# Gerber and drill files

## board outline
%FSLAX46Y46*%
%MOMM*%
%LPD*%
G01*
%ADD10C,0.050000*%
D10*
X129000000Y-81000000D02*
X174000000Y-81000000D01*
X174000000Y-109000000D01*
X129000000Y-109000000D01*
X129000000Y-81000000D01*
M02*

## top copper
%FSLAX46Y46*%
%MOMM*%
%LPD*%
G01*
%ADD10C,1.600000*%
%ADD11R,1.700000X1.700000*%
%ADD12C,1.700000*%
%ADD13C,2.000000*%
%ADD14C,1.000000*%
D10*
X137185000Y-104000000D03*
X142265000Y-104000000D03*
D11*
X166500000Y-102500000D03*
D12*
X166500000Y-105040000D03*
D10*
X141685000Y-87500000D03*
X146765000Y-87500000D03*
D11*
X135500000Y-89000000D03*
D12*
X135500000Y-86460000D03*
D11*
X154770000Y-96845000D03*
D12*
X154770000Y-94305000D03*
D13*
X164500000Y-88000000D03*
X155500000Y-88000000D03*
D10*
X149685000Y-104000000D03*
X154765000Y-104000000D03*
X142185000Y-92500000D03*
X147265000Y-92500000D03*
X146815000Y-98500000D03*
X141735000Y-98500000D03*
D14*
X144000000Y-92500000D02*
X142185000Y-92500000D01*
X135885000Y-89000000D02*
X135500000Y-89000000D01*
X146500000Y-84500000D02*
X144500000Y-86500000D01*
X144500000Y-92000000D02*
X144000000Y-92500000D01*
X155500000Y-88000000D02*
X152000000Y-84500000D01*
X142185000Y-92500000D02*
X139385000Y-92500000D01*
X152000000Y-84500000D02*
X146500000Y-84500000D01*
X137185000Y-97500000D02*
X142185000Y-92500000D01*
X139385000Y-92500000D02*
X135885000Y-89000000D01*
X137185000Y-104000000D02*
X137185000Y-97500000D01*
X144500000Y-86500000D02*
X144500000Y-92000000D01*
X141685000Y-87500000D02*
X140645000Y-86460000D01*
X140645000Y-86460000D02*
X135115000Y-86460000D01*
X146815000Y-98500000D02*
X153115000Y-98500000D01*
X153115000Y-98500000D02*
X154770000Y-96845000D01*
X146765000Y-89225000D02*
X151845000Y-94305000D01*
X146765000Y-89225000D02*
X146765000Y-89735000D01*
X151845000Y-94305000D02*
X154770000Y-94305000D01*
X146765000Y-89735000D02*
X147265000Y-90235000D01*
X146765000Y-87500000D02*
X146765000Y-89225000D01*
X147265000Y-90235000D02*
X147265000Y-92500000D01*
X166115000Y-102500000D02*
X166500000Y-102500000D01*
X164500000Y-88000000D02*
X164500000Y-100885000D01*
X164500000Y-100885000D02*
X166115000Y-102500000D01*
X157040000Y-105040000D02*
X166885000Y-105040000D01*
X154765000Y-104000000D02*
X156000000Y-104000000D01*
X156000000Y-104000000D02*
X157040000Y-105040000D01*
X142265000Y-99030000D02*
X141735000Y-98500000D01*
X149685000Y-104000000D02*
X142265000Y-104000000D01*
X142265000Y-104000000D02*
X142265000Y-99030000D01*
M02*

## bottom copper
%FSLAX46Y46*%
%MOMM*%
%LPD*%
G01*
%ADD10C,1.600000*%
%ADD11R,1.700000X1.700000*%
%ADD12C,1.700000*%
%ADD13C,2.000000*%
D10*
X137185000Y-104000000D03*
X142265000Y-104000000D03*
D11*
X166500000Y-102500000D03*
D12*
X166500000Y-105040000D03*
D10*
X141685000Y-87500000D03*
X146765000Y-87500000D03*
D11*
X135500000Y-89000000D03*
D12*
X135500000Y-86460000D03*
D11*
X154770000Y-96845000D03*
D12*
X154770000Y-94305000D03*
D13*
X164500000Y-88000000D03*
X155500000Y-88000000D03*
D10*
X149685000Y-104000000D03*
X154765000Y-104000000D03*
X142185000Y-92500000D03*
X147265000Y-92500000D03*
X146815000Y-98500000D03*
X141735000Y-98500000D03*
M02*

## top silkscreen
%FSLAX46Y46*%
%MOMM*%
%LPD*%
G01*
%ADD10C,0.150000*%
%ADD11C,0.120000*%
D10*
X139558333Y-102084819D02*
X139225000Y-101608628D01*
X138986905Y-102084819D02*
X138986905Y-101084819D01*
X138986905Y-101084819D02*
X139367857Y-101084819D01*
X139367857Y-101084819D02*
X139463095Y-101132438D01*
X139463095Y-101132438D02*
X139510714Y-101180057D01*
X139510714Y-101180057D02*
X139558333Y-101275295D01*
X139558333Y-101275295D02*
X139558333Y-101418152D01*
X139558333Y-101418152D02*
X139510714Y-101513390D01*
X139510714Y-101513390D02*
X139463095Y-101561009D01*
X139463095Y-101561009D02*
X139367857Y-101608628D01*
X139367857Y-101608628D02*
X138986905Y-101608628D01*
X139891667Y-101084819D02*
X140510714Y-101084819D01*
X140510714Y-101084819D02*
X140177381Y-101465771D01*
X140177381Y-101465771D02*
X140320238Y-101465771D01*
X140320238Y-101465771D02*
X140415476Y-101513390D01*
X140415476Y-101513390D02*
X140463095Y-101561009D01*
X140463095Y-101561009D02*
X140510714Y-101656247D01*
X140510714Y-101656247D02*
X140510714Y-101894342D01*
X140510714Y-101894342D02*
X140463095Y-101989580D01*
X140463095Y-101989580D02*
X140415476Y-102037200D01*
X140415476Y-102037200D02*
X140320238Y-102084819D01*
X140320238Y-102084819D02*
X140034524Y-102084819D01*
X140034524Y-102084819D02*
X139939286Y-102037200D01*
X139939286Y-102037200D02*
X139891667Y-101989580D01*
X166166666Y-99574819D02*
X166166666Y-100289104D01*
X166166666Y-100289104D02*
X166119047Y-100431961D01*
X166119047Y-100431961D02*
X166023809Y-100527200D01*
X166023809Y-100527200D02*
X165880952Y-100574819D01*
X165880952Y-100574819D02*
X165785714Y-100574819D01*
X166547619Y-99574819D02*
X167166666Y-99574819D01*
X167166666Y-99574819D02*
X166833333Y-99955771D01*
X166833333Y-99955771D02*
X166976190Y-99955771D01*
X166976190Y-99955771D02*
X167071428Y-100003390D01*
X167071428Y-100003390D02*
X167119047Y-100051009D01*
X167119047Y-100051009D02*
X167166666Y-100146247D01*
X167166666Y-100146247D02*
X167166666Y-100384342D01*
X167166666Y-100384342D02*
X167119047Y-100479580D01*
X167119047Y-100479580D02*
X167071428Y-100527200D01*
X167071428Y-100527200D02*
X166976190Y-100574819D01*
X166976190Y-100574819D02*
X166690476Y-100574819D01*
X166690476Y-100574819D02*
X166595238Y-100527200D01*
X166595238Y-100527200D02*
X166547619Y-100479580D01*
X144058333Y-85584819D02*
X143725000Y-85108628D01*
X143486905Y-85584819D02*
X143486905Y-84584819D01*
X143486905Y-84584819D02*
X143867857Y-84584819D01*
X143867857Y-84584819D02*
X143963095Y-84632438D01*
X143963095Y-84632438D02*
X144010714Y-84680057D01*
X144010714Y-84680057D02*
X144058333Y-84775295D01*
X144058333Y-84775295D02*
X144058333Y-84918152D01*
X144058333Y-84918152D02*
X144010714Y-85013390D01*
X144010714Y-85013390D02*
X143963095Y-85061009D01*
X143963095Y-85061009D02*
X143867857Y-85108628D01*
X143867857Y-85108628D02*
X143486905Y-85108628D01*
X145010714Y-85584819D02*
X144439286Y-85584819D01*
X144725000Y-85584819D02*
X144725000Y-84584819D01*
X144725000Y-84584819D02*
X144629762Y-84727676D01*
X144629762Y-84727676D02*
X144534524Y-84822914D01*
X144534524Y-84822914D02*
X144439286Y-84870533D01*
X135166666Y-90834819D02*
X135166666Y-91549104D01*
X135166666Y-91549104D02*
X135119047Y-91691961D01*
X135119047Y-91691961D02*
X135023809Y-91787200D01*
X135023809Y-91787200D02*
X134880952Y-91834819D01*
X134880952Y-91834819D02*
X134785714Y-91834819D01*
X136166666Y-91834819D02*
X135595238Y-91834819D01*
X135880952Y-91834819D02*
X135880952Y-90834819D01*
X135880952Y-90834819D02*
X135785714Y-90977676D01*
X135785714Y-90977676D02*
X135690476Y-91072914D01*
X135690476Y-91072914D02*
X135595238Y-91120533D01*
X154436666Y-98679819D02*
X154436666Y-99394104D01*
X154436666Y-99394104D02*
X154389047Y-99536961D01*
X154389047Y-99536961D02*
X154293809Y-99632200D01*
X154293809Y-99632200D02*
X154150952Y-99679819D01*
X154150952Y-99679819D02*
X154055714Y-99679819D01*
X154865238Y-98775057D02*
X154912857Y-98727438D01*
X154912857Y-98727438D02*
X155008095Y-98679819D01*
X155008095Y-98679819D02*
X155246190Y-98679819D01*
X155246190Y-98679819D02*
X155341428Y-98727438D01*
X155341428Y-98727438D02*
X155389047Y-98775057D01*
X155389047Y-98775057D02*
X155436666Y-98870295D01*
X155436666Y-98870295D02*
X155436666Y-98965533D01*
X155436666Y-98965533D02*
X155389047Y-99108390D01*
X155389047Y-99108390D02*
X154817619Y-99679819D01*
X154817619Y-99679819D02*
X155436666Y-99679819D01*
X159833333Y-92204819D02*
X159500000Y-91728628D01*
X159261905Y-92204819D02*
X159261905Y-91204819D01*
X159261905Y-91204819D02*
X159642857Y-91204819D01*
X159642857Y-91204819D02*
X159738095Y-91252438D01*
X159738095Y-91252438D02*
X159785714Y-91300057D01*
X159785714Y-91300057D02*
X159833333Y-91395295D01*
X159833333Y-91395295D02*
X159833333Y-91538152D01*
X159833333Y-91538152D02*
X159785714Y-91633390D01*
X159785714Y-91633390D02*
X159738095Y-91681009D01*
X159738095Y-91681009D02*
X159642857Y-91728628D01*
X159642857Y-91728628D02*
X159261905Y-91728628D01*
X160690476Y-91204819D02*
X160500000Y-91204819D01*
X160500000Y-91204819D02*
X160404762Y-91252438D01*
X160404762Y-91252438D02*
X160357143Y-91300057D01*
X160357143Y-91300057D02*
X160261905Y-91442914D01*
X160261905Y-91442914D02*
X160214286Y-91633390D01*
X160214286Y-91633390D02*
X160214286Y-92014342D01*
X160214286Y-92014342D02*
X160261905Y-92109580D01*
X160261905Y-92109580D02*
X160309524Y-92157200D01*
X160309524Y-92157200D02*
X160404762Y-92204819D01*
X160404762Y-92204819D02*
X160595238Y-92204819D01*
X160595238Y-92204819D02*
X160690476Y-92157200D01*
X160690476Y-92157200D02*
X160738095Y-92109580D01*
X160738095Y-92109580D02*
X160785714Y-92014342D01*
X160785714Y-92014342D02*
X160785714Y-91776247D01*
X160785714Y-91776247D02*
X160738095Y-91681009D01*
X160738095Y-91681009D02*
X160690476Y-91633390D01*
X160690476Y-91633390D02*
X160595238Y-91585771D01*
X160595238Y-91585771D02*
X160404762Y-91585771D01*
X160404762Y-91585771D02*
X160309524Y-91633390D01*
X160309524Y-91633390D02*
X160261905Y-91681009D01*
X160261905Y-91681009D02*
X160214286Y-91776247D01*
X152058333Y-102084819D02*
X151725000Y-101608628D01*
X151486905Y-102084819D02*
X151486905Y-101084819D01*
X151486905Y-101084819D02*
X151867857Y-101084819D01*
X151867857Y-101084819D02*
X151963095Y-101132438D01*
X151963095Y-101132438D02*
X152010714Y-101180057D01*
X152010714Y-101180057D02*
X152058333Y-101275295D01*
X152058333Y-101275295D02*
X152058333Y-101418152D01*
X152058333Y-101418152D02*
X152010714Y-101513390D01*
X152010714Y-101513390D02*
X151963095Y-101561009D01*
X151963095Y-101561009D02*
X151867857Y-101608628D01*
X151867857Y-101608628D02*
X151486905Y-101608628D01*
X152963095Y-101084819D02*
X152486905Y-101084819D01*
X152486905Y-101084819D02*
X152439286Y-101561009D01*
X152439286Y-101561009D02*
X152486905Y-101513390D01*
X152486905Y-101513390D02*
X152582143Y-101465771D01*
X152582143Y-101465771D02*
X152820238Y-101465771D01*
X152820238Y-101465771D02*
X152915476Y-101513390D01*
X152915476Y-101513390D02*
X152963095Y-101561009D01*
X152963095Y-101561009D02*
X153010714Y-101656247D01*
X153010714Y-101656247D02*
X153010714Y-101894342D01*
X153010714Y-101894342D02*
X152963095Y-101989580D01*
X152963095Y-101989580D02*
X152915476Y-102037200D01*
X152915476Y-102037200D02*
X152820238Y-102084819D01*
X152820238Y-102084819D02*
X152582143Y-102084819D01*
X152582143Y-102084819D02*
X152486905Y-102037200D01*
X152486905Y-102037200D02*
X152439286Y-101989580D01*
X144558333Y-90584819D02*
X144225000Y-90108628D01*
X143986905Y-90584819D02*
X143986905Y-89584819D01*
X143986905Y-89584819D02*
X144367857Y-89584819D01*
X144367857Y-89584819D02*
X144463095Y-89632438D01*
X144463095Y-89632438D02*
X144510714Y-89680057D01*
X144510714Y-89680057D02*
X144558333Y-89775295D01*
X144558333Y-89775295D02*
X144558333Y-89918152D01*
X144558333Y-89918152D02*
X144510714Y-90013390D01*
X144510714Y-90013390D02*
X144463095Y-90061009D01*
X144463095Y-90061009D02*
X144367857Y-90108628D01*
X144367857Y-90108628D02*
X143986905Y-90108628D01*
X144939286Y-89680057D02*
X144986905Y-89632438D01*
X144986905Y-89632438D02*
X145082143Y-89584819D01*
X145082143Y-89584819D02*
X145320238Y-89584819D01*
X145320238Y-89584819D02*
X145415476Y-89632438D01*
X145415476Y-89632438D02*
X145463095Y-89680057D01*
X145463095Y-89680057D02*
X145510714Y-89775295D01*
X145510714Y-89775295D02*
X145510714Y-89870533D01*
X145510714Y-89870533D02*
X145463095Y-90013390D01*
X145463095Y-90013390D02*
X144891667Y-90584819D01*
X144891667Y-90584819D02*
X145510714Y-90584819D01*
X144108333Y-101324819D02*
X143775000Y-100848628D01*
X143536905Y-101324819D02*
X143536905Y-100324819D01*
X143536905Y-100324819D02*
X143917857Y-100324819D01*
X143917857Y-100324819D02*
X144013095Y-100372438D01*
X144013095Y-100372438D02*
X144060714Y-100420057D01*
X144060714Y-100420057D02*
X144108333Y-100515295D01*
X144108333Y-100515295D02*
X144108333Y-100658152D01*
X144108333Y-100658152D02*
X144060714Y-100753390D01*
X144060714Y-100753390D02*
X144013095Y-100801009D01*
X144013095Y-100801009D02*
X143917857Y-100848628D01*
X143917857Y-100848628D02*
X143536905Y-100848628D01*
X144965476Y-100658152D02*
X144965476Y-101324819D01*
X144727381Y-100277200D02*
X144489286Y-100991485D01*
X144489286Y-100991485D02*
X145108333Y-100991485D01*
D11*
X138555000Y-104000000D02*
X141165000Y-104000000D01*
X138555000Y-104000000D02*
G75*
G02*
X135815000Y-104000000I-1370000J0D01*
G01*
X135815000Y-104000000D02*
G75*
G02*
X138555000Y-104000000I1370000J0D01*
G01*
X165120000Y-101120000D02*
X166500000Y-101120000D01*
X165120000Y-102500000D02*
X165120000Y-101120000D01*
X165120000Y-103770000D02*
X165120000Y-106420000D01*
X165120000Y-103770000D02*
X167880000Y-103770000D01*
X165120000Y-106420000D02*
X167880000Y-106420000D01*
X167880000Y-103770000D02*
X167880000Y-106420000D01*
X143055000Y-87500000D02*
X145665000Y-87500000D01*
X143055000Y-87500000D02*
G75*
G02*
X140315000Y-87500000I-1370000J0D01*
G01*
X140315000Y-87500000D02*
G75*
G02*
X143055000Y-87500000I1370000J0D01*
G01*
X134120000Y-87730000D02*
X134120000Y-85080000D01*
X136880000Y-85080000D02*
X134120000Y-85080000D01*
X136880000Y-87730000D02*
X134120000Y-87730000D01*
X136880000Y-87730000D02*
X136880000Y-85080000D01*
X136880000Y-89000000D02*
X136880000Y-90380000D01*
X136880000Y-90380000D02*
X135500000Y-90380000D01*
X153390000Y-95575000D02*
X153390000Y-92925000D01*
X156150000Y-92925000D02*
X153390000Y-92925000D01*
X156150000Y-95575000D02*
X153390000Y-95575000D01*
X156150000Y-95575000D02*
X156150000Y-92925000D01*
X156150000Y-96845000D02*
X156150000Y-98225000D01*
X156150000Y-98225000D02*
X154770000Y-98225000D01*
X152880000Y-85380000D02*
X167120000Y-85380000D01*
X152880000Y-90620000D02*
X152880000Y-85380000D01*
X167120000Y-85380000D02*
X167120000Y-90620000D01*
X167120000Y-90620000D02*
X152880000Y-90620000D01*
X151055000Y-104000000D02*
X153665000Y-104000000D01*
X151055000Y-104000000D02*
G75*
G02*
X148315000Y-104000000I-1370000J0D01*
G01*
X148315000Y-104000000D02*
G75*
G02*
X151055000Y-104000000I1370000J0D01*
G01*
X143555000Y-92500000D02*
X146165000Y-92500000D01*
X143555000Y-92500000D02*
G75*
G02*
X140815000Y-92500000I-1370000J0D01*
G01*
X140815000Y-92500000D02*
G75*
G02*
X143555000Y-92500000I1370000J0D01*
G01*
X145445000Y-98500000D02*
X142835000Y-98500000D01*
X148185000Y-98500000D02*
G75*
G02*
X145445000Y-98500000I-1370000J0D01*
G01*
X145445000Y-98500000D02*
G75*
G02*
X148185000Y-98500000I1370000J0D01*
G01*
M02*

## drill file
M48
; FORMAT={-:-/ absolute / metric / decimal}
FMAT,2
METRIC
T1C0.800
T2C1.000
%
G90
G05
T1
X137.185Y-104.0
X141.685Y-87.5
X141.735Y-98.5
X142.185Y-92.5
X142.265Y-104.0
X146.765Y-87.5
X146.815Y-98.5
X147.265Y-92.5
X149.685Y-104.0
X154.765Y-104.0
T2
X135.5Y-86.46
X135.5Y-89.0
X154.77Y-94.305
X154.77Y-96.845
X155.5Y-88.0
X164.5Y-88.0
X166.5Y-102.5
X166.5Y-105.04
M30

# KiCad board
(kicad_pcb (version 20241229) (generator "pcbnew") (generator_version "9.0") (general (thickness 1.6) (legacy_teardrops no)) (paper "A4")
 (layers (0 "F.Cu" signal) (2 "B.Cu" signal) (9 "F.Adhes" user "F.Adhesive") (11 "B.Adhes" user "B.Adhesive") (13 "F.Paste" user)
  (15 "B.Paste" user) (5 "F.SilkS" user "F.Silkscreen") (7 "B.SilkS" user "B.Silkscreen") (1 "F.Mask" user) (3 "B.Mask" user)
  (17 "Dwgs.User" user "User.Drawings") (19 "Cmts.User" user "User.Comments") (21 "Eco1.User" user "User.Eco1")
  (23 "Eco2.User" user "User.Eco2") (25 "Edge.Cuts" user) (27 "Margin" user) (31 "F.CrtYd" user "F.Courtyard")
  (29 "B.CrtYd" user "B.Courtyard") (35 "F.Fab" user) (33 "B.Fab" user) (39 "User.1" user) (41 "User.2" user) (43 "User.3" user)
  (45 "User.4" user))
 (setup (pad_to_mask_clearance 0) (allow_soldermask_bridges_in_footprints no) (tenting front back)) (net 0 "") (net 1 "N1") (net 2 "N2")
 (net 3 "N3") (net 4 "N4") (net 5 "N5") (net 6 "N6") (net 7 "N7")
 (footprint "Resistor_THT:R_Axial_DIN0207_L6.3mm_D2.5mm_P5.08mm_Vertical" (layer "F.Cu") (at 137.185 104)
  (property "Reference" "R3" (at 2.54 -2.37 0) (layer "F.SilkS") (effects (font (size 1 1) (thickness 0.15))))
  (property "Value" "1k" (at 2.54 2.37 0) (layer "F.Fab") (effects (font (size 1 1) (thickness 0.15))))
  (fp_line (start 1.37 0) (end 3.98 0) (stroke (width 0.12) (type solid)) (layer "F.SilkS"))
  (fp_circle (center 0 0) (end 1.37 0) (stroke (width 0.12) (type solid)) (fill no) (layer "F.SilkS"))
  (pad "1" thru_hole circle (at 0 0) (size 1.6 1.6) (drill 0.8) (layers "*.Cu" "*.Mask") (remove_unused_layers no) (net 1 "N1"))
  (pad "2" thru_hole circle (at 5.08 0) (size 1.6 1.6) (drill 0.8) (layers "*.Cu" "*.Mask") (remove_unused_layers no) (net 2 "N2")))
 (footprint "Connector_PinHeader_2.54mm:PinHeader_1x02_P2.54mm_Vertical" (layer "F.Cu") (at 166.5 102.5)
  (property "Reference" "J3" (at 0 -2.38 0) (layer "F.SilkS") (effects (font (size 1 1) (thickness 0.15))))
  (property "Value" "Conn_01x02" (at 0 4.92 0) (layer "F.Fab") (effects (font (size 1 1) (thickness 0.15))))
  (fp_line (start -1.38 -1.38) (end 0 -1.38) (stroke (width 0.12) (type solid)) (layer "F.SilkS"))
  (fp_line (start -1.38 0) (end -1.38 -1.38) (stroke (width 0.12) (type solid)) (layer "F.SilkS"))
  (fp_line (start -1.38 1.27) (end -1.38 3.92) (stroke (width 0.12) (type solid)) (layer "F.SilkS"))
  (fp_line (start -1.38 1.27) (end 1.38 1.27) (stroke (width 0.12) (type solid)) (layer "F.SilkS"))
  (fp_line (start -1.38 3.92) (end 1.38 3.92) (stroke (width 0.12) (type solid)) (layer "F.SilkS"))
  (fp_line (start 1.38 1.27) (end 1.38 3.92) (stroke (width 0.12) (type solid)) (layer "F.SilkS"))
  (pad "1" thru_hole rect (at 0 0) (size 1.7 1.7) (drill 1) (layers "*.Cu" "*.Mask") (remove_unused_layers no) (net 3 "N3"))
  (pad "2" thru_hole circle (at 0 2.54) (size 1.7 1.7) (drill 1) (layers "*.Cu" "*.Mask") (remove_unused_layers no) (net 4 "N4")))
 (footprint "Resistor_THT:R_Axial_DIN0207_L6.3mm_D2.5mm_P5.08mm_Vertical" (layer "F.Cu") (at 141.685 87.5)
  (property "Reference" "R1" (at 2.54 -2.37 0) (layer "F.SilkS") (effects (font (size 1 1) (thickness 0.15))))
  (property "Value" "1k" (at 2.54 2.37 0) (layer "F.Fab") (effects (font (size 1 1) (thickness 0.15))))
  (fp_line (start 1.37 0) (end 3.98 0) (stroke (width 0.12) (type solid)) (layer "F.SilkS"))
  (fp_circle (center 0 0) (end 1.37 0) (stroke (width 0.12) (type solid)) (fill no) (layer "F.SilkS"))
  (pad "1" thru_hole circle (at 0 0) (size 1.6 1.6) (drill 0.8) (layers "*.Cu" "*.Mask") (remove_unused_layers no) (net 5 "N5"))
  (pad "2" thru_hole circle (at 5.08 0) (size 1.6 1.6) (drill 0.8) (layers "*.Cu" "*.Mask") (remove_unused_layers no) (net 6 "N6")))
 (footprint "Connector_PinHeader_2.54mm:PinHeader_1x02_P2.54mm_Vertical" (layer "F.Cu") (at 135.5 89 180)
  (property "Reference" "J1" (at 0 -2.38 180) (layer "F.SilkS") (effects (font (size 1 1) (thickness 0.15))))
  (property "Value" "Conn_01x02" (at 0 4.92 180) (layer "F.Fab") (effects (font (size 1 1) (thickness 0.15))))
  (fp_line (start 1.38 1.27) (end 1.38 3.92) (stroke (width 0.12) (type solid)) (layer "F.SilkS"))
  (fp_line (start -1.38 3.92) (end 1.38 3.92) (stroke (width 0.12) (type solid)) (layer "F.SilkS"))
  (fp_line (start -1.38 1.27) (end 1.38 1.27) (stroke (width 0.12) (type solid)) (layer "F.SilkS"))
  (fp_line (start -1.38 1.27) (end -1.38 3.92) (stroke (width 0.12) (type solid)) (layer "F.SilkS"))
  (fp_line (start -1.38 0) (end -1.38 -1.38) (stroke (width 0.12) (type solid)) (layer "F.SilkS"))
  (fp_line (start -1.38 -1.38) (end 0 -1.38) (stroke (width 0.12) (type solid)) (layer "F.SilkS"))
  (pad "1" thru_hole rect (at 0 0 180) (size 1.7 1.7) (drill 1) (layers "*.Cu" "*.Mask") (remove_unused_layers no) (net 1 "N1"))
  (pad "2" thru_hole circle (at 0 2.54 180) (size 1.7 1.7) (drill 1) (layers "*.Cu" "*.Mask") (remove_unused_layers no) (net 5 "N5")))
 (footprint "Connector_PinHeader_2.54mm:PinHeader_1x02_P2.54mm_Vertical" (layer "F.Cu") (at 154.77 96.845 180)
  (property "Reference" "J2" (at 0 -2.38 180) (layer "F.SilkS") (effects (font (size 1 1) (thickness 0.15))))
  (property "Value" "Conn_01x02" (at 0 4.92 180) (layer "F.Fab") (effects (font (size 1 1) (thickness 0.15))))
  (fp_line (start 1.38 1.27) (end 1.38 3.92) (stroke (width 0.12) (type solid)) (layer "F.SilkS"))
  (fp_line (start -1.38 3.92) (end 1.38 3.92) (stroke (width 0.12) (type solid)) (layer "F.SilkS"))
  (fp_line (start -1.38 1.27) (end 1.38 1.27) (stroke (width 0.12) (type solid)) (layer "F.SilkS"))
  (fp_line (start -1.38 1.27) (end -1.38 3.92) (stroke (width 0.12) (type solid)) (layer "F.SilkS"))
  (fp_line (start -1.38 0) (end -1.38 -1.38) (stroke (width 0.12) (type solid)) (layer "F.SilkS"))
  (fp_line (start -1.38 -1.38) (end 0 -1.38) (stroke (width 0.12) (type solid)) (layer "F.SilkS"))
  (pad "1" thru_hole rect (at 0 0 180) (size 1.7 1.7) (drill 1) (layers "*.Cu" "*.Mask") (remove_unused_layers no) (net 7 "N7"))
  (pad "2" thru_hole circle (at 0 2.54 180) (size 1.7 1.7) (drill 1) (layers "*.Cu" "*.Mask") (remove_unused_layers no) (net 6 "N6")))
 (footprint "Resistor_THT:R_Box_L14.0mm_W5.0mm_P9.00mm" (layer "F.Cu") (at 164.5 88 180)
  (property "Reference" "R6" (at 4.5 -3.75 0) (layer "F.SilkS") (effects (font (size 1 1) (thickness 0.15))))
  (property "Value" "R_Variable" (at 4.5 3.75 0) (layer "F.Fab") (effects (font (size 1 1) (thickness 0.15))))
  (fp_line (start 11.62 2.62) (end -2.62 2.62) (stroke (width 0.12) (type solid)) (layer "F.SilkS"))
  (fp_line (start 11.62 -2.62) (end 11.62 2.62) (stroke (width 0.12) (type solid)) (layer "F.SilkS"))
  (fp_line (start -2.62 2.62) (end -2.62 -2.62) (stroke (width 0.12) (type solid)) (layer "F.SilkS"))
  (fp_line (start -2.62 -2.62) (end 11.62 -2.62) (stroke (width 0.12) (type solid)) (layer "F.SilkS"))
  (pad "1" thru_hole circle (at 0 0 180) (size 2 2) (drill 1) (layers "*.Cu" "*.Mask") (remove_unused_layers no) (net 3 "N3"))
  (pad "2" thru_hole circle (at 9 0 180) (size 2 2) (drill 1) (layers "*.Cu" "*.Mask") (remove_unused_layers no) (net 1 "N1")))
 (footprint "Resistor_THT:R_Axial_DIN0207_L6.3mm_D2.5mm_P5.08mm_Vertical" (layer "F.Cu") (at 149.685 104)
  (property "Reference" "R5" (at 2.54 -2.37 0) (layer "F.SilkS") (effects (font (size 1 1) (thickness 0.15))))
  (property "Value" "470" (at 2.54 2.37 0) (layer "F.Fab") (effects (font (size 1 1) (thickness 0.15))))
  (fp_line (start 1.37 0) (end 3.98 0) (stroke (width 0.12) (type solid)) (layer "F.SilkS"))
  (fp_circle (center 0 0) (end 1.37 0) (stroke (width 0.12) (type solid)) (fill no) (layer "F.SilkS"))
  (pad "1" thru_hole circle (at 0 0) (size 1.6 1.6) (drill 0.8) (layers "*.Cu" "*.Mask") (remove_unused_layers no) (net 2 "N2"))
  (pad "2" thru_hole circle (at 5.08 0) (size 1.6 1.6) (drill 0.8) (layers "*.Cu" "*.Mask") (remove_unused_layers no) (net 4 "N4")))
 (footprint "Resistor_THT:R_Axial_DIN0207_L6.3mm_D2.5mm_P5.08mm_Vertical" (layer "F.Cu") (at 142.185 92.5)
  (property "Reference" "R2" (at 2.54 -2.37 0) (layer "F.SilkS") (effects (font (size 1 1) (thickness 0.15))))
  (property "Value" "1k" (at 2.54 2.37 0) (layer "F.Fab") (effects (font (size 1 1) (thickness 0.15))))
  (fp_line (start 1.37 0) (end 3.98 0) (stroke (width 0.12) (type solid)) (layer "F.SilkS"))
  (fp_circle (center 0 0) (end 1.37 0) (stroke (width 0.12) (type solid)) (fill no) (layer "F.SilkS"))
  (pad "1" thru_hole circle (at 0 0) (size 1.6 1.6) (drill 0.8) (layers "*.Cu" "*.Mask") (remove_unused_layers no) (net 1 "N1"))
  (pad "2" thru_hole circle (at 5.08 0) (size 1.6 1.6) (drill 0.8) (layers "*.Cu" "*.Mask") (remove_unused_layers no) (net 6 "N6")))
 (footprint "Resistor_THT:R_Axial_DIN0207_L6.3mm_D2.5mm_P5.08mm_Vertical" (layer "F.Cu") (at 146.815 98.5 180)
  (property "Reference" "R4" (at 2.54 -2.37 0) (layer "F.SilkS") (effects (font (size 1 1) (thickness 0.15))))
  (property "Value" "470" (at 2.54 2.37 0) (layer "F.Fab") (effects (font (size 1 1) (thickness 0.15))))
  (fp_line (start 1.37 0) (end 3.98 0) (stroke (width 0.12) (type solid)) (layer "F.SilkS"))
  (fp_circle (center 0 0) (end 1.37 0) (stroke (width 0.12) (type solid)) (fill no) (layer "F.SilkS"))
  (pad "1" thru_hole circle (at 0 0 180) (size 1.6 1.6) (drill 0.8) (layers "*.Cu" "*.Mask") (remove_unused_layers no) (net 7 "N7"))
  (pad "2" thru_hole circle (at 5.08 0 180) (size 1.6 1.6) (drill 0.8) (layers "*.Cu" "*.Mask") (remove_unused_layers no) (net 2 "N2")))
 (gr_rect (start 129 81) (end 174 109) (stroke (width 0.05) (type default)) (fill no) (layer "Edge.Cuts"))
 (segment (start 144 92.5) (end 142.185 92.5) (width 1) (layer "F.Cu") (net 1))
 (segment (start 135.885 89) (end 135.5 89) (width 1) (layer "F.Cu") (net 1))
 (segment (start 146.5 84.5) (end 144.5 86.5) (width 1) (layer "F.Cu") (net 1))
 (segment (start 144.5 92) (end 144 92.5) (width 1) (layer "F.Cu") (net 1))
 (segment (start 155.5 88) (end 152 84.5) (width 1) (layer "F.Cu") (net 1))
 (segment (start 142.185 92.5) (end 139.385 92.5) (width 1) (layer "F.Cu") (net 1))
 (segment (start 152 84.5) (end 146.5 84.5) (width 1) (layer "F.Cu") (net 1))
 (segment (start 137.185 97.5) (end 142.185 92.5) (width 1) (layer "F.Cu") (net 1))
 (segment (start 139.385 92.5) (end 135.885 89) (width 1) (layer "F.Cu") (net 1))
 (segment (start 137.185 104) (end 137.185 97.5) (width 1) (layer "F.Cu") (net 1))
 (segment (start 144.5 86.5) (end 144.5 92) (width 1) (layer "F.Cu") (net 1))
 (segment (start 141.685 87.5) (end 140.645 86.46) (width 1) (layer "F.Cu") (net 5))
 (segment (start 140.645 86.46) (end 135.115 86.46) (width 1) (layer "F.Cu") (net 5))
 (segment (start 146.815 98.5) (end 153.115 98.5) (width 1) (layer "F.Cu") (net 7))
 (segment (start 153.115 98.5) (end 154.77 96.845) (width 1) (layer "F.Cu") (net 7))
 (segment (start 146.765 89.225) (end 151.845 94.305) (width 1) (layer "F.Cu") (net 6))
 (segment (start 146.765 89.225) (end 146.765 89.735) (width 1) (layer "F.Cu") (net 6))
 (segment (start 151.845 94.305) (end 154.77 94.305) (width 1) (layer "F.Cu") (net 6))
 (segment (start 146.765 89.735) (end 147.265 90.235) (width 1) (layer "F.Cu") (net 6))
 (segment (start 146.765 87.5) (end 146.765 89.225) (width 1) (layer "F.Cu") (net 6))
 (segment (start 147.265 90.235) (end 147.265 92.5) (width 1) (layer "F.Cu") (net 6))
 (segment (start 166.115 102.5) (end 166.5 102.5) (width 1) (layer "F.Cu") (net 3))
 (segment (start 164.5 88) (end 164.5 100.885) (width 1) (layer "F.Cu") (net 3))
 (segment (start 164.5 100.885) (end 166.115 102.5) (width 1) (layer "F.Cu") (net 3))
 (segment (start 157.04 105.04) (end 166.885 105.04) (width 1) (layer "F.Cu") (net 4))
 (segment (start 154.765 104) (end 156 104) (width 1) (layer "F.Cu") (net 4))
 (segment (start 156 104) (end 157.04 105.04) (width 1) (layer "F.Cu") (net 4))
 (segment (start 142.265 99.03) (end 141.735 98.5) (width 1) (layer "F.Cu") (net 2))
 (segment (start 149.685 104) (end 142.265 104) (width 1) (layer "F.Cu") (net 2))
 (segment (start 142.265 104) (end 142.265 99.03) (width 1) (layer "F.Cu") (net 2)))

